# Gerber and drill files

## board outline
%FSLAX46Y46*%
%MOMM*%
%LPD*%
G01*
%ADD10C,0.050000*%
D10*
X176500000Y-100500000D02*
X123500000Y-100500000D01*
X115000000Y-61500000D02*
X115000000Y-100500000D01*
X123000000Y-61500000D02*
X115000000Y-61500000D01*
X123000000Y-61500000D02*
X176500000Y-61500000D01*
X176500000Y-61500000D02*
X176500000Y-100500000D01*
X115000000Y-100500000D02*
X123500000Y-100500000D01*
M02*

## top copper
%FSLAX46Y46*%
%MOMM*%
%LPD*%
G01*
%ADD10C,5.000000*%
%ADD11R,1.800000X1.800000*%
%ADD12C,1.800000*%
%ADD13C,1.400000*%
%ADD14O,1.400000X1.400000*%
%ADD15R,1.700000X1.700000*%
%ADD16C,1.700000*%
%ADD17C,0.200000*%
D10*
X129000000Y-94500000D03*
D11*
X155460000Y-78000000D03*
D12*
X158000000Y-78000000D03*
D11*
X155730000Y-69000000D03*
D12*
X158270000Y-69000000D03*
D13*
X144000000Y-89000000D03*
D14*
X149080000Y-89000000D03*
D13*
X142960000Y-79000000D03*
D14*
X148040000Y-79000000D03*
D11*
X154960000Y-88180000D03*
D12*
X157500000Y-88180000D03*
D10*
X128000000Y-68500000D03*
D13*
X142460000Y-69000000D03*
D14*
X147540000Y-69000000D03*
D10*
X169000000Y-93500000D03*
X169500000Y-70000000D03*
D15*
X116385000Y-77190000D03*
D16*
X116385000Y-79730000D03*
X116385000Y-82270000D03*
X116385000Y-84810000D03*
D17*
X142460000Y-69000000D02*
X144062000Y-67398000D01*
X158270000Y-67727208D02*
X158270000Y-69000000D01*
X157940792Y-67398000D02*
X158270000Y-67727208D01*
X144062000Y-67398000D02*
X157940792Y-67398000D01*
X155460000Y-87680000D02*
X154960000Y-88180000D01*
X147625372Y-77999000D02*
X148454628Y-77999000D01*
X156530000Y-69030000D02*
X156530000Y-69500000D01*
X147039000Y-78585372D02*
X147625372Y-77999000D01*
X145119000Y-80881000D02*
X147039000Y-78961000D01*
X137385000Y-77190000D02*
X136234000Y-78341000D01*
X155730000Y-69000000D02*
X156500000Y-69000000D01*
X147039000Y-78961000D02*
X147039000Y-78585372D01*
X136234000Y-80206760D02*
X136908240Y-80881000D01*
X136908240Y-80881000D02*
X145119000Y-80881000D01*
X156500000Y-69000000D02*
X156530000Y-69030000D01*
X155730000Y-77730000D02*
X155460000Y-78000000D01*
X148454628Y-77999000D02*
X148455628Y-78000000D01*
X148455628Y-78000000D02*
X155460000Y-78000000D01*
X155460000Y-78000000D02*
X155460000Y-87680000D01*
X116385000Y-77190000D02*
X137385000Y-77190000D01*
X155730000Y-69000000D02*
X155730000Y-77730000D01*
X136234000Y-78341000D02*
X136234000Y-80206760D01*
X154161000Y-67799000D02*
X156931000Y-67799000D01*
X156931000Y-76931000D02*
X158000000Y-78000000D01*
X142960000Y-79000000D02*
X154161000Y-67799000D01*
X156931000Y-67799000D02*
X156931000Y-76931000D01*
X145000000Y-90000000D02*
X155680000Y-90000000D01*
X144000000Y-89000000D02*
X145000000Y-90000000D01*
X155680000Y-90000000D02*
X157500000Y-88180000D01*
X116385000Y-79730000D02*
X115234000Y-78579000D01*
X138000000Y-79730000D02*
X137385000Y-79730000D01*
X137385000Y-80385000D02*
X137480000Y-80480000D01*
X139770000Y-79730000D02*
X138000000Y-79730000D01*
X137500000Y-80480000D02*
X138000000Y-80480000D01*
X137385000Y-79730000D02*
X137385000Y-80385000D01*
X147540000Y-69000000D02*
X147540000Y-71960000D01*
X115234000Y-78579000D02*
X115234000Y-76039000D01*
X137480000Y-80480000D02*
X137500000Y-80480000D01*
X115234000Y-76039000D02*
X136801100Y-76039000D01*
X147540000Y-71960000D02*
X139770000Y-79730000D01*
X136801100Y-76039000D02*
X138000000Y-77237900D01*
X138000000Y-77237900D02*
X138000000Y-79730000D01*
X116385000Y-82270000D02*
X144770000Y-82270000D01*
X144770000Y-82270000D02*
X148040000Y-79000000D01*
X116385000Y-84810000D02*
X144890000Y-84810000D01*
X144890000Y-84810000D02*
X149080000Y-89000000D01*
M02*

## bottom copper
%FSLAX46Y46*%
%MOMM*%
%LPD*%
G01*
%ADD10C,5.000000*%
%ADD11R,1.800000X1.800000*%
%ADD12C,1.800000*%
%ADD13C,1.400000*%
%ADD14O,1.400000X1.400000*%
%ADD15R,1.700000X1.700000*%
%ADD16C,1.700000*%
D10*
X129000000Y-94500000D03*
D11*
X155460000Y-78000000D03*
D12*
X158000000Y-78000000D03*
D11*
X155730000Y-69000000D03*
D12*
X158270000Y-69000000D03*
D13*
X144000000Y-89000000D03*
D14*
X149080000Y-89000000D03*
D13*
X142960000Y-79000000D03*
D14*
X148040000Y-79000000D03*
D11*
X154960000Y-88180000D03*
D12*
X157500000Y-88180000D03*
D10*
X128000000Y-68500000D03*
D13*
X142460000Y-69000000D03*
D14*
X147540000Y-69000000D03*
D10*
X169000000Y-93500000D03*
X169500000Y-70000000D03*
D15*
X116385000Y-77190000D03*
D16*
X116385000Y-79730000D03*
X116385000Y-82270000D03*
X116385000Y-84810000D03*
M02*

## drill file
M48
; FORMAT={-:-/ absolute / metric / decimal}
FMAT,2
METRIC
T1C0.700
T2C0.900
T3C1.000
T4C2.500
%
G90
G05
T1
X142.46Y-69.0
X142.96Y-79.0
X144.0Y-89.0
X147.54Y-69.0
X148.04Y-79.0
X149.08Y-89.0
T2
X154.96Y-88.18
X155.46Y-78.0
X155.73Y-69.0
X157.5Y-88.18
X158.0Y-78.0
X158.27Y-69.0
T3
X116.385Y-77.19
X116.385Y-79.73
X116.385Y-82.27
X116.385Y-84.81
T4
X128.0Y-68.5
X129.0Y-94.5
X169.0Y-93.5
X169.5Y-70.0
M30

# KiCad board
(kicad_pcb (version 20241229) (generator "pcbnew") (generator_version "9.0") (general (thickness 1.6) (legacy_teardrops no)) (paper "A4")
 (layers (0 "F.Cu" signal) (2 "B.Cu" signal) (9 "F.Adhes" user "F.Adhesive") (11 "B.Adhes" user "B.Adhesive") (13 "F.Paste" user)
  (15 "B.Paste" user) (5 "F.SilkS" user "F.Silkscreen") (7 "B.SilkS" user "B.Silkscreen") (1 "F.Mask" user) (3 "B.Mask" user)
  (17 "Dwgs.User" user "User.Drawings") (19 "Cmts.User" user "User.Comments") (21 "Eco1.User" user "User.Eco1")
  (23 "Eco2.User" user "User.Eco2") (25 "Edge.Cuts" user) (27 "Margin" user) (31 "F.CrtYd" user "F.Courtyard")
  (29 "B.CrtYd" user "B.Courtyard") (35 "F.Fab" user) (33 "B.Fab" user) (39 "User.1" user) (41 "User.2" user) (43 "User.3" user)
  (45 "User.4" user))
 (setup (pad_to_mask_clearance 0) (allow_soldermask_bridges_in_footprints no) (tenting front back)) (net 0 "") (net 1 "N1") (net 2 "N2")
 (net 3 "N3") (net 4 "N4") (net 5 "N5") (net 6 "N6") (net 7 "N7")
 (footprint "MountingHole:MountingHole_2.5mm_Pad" (layer "F.Cu") (at 129 94.5)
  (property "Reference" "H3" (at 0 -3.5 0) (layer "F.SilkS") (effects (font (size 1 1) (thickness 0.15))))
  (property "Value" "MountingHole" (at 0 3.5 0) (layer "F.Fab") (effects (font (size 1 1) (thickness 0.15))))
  (pad "1" thru_hole circle (at 0 0) (size 5 5) (drill 2.5) (layers "*.Cu" "*.Mask") (remove_unused_layers no)))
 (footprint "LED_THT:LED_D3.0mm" (layer "F.Cu") (at 155.46 78)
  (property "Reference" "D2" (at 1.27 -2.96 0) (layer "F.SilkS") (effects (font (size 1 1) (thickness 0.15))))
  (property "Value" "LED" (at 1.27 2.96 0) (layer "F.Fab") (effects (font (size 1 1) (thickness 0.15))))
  (pad "1" thru_hole rect (at 0 0) (size 1.8 1.8) (drill 0.9) (layers "*.Cu" "*.Mask") (remove_unused_layers no) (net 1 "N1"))
  (pad "2" thru_hole circle (at 2.54 0) (size 1.8 1.8) (drill 0.9) (layers "*.Cu" "*.Mask") (remove_unused_layers no) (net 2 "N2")))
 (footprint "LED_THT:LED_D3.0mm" (layer "F.Cu") (at 155.73 69)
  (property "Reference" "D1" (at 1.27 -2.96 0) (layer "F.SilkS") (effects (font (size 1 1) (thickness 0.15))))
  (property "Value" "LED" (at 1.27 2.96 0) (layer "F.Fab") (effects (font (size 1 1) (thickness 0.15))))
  (pad "1" thru_hole rect (at 0 0) (size 1.8 1.8) (drill 0.9) (layers "*.Cu" "*.Mask") (remove_unused_layers no) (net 1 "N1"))
  (pad "2" thru_hole circle (at 2.54 0) (size 1.8 1.8) (drill 0.9) (layers "*.Cu" "*.Mask") (remove_unused_layers no) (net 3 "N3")))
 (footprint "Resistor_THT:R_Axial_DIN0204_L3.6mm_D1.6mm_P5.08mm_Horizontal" (layer "F.Cu") (at 144 89)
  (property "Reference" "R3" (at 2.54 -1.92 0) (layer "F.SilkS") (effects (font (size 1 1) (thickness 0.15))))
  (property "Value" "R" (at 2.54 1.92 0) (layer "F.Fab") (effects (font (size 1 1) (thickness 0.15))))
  (pad "1" thru_hole circle (at 0 0) (size 1.4 1.4) (drill 0.7) (layers "*.Cu" "*.Mask") (remove_unused_layers no) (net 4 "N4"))
  (pad "2" thru_hole oval (at 5.08 0) (size 1.4 1.4) (drill 0.7) (layers "*.Cu" "*.Mask") (remove_unused_layers no) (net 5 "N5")))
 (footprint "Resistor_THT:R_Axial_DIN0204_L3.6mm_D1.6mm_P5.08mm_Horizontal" (layer "F.Cu") (at 142.96 79)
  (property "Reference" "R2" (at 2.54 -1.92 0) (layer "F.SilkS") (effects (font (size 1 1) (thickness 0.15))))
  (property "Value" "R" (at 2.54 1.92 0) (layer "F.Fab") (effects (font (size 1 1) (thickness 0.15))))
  (pad "1" thru_hole circle (at 0 0) (size 1.4 1.4) (drill 0.7) (layers "*.Cu" "*.Mask") (remove_unused_layers no) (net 2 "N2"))
  (pad "2" thru_hole oval (at 5.08 0) (size 1.4 1.4) (drill 0.7) (layers "*.Cu" "*.Mask") (remove_unused_layers no) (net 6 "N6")))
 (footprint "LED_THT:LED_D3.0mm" (layer "F.Cu") (at 154.96 88.18)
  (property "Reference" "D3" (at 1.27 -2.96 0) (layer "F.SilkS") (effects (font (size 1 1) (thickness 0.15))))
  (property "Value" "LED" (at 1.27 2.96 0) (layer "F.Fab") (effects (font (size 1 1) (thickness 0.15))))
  (pad "1" thru_hole rect (at 0 0) (size 1.8 1.8) (drill 0.9) (layers "*.Cu" "*.Mask") (remove_unused_layers no) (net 1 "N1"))
  (pad "2" thru_hole circle (at 2.54 0) (size 1.8 1.8) (drill 0.9) (layers "*.Cu" "*.Mask") (remove_unused_layers no) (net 4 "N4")))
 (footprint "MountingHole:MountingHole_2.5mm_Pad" (layer "F.Cu") (at 128 68.5)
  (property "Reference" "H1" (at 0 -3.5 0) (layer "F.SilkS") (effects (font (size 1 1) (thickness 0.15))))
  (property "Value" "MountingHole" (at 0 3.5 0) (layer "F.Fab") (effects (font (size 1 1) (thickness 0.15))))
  (pad "1" thru_hole circle (at 0 0) (size 5 5) (drill 2.5) (layers "*.Cu" "*.Mask") (remove_unused_layers no)))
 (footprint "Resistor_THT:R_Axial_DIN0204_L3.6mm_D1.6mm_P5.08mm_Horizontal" (layer "F.Cu") (at 142.46 69)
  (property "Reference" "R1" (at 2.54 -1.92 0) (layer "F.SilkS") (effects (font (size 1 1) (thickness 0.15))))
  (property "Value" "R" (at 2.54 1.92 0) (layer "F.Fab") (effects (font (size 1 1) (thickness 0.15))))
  (pad "1" thru_hole circle (at 0 0) (size 1.4 1.4) (drill 0.7) (layers "*.Cu" "*.Mask") (remove_unused_layers no) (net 3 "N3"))
  (pad "2" thru_hole oval (at 5.08 0) (size 1.4 1.4) (drill 0.7) (layers "*.Cu" "*.Mask") (remove_unused_layers no) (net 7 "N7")))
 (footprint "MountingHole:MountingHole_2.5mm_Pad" (layer "F.Cu") (at 169 93.5)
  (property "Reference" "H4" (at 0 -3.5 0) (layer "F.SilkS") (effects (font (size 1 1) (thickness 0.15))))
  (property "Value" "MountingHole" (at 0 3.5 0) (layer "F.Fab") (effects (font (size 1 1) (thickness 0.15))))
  (pad "1" thru_hole circle (at 0 0) (size 5 5) (drill 2.5) (layers "*.Cu" "*.Mask") (remove_unused_layers no)))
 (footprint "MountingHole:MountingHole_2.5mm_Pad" (layer "F.Cu") (at 169.5 70)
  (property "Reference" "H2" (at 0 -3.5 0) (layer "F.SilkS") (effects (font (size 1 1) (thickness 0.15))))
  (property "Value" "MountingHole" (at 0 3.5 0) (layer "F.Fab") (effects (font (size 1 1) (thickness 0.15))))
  (pad "1" thru_hole circle (at 0 0) (size 5 5) (drill 2.5) (layers "*.Cu" "*.Mask") (remove_unused_layers no)))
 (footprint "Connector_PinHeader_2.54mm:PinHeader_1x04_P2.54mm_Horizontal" (layer "B.Cu") (at 116.385 77.19 180)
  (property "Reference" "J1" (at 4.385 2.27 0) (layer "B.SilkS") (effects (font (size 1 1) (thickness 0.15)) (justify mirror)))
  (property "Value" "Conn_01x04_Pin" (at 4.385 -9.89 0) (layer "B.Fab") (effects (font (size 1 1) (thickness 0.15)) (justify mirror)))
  (pad "1" thru_hole rect (at 0 0 180) (size 1.7 1.7) (drill 1) (layers "*.Cu" "*.Mask") (remove_unused_layers no) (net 1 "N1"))
  (pad "2" thru_hole circle (at 0 -2.54 180) (size 1.7 1.7) (drill 1) (layers "*.Cu" "*.Mask") (remove_unused_layers no) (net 7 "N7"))
  (pad "3" thru_hole circle (at 0 -5.08 180) (size 1.7 1.7) (drill 1) (layers "*.Cu" "*.Mask") (remove_unused_layers no) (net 6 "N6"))
  (pad "4" thru_hole circle (at 0 -7.62 180) (size 1.7 1.7) (drill 1) (layers "*.Cu" "*.Mask") (remove_unused_layers no) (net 5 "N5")))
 (gr_line (start 176.5 100.5) (end 123.5 100.5) (stroke (width 0.05) (type default)) (layer "Edge.Cuts"))
 (gr_line (start 115 61.5) (end 115 100.5) (stroke (width 0.05) (type default)) (layer "Edge.Cuts"))
 (gr_line (start 123 61.5) (end 115 61.5) (stroke (width 0.05) (type default)) (layer "Edge.Cuts"))
 (gr_line (start 123 61.5) (end 176.5 61.5) (stroke (width 0.05) (type default)) (layer "Edge.Cuts"))
 (gr_line (start 176.5 61.5) (end 176.5 100.5) (stroke (width 0.05) (type default)) (layer "Edge.Cuts"))
 (gr_line (start 115 100.5) (end 123.5 100.5) (stroke (width 0.05) (type default)) (layer "Edge.Cuts"))
 (segment (start 142.46 69) (end 144.062 67.398) (width 0.2) (layer "F.Cu") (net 3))
 (segment (start 158.27 67.727208) (end 158.27 69) (width 0.2) (layer "F.Cu") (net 3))
 (segment (start 157.940792 67.398) (end 158.27 67.727208) (width 0.2) (layer "F.Cu") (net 3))
 (segment (start 144.062 67.398) (end 157.940792 67.398) (width 0.2) (layer "F.Cu") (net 3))
 (segment (start 155.46 87.68) (end 154.96 88.18) (width 0.2) (layer "F.Cu") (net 1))
 (segment (start 147.625372 77.999) (end 148.454628 77.999) (width 0.2) (layer "F.Cu") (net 1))
 (segment (start 156.53 69.03) (end 156.53 69.5) (width 0.2) (layer "F.Cu") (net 1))
 (segment (start 147.039 78.585372) (end 147.625372 77.999) (width 0.2) (layer "F.Cu") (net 1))
 (segment (start 145.119 80.881) (end 147.039 78.961) (width 0.2) (layer "F.Cu") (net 1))
 (segment (start 137.385 77.19) (end 136.234 78.341) (width 0.2) (layer "F.Cu") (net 1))
 (segment (start 155.73 69) (end 156.5 69) (width 0.2) (layer "F.Cu") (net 1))
 (segment (start 147.039 78.961) (end 147.039 78.585372) (width 0.2) (layer "F.Cu") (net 1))
 (segment (start 136.234 80.20676) (end 136.90824 80.881) (width 0.2) (layer "F.Cu") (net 1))
 (segment (start 136.90824 80.881) (end 145.119 80.881) (width 0.2) (layer "F.Cu") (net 1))
 (segment (start 156.5 69) (end 156.53 69.03) (width 0.2) (layer "F.Cu") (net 1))
 (segment (start 155.73 77.73) (end 155.46 78) (width 0.2) (layer "F.Cu") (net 1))
 (segment (start 148.454628 77.999) (end 148.455628 78) (width 0.2) (layer "F.Cu") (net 1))
 (segment (start 148.455628 78) (end 155.46 78) (width 0.2) (layer "F.Cu") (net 1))
 (segment (start 155.46 78) (end 155.46 87.68) (width 0.2) (layer "F.Cu") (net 1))
 (segment (start 116.385 77.19) (end 137.385 77.19) (width 0.2) (layer "F.Cu") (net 1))
 (segment (start 155.73 69) (end 155.73 77.73) (width 0.2) (layer "F.Cu") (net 1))
 (segment (start 136.234 78.341) (end 136.234 80.20676) (width 0.2) (layer "F.Cu") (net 1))
 (segment (start 154.161 67.799) (end 156.931 67.799) (width 0.2) (layer "F.Cu") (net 2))
 (segment (start 156.931 76.931) (end 158 78) (width 0.2) (layer "F.Cu") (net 2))
 (segment (start 142.96 79) (end 154.161 67.799) (width 0.2) (layer "F.Cu") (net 2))
 (segment (start 156.931 67.799) (end 156.931 76.931) (width 0.2) (layer "F.Cu") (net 2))
 (segment (start 145 90) (end 155.68 90) (width 0.2) (layer "F.Cu") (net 4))
 (segment (start 144 89) (end 145 90) (width 0.2) (layer "F.Cu") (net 4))
 (segment (start 155.68 90) (end 157.5 88.18) (width 0.2) (layer "F.Cu") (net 4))
 (segment (start 116.385 79.73) (end 115.234 78.579) (width 0.2) (layer "F.Cu") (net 7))
 (segment (start 138 79.73) (end 137.385 79.73) (width 0.2) (layer "F.Cu") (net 7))
 (segment (start 137.385 80.385) (end 137.48 80.48) (width 0.2) (layer "F.Cu") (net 7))
 (segment (start 139.77 79.73) (end 138 79.73) (width 0.2) (layer "F.Cu") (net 7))
 (segment (start 137.5 80.48) (end 138 80.48) (width 0.2) (layer "F.Cu") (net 7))
 (segment (start 137.385 79.73) (end 137.385 80.385) (width 0.2) (layer "F.Cu") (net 7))
 (segment (start 147.54 69) (end 147.54 71.96) (width 0.2) (layer "F.Cu") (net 7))
 (segment (start 115.234 78.579) (end 115.234 76.039) (width 0.2) (layer "F.Cu") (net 7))
 (segment (start 137.48 80.48) (end 137.5 80.48) (width 0.2) (layer "F.Cu") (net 7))
 (segment (start 115.234 76.039) (end 136.8011 76.039) (width 0.2) (layer "F.Cu") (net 7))
 (segment (start 147.54 71.96) (end 139.77 79.73) (width 0.2) (layer "F.Cu") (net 7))
 (segment (start 136.8011 76.039) (end 138 77.2379) (width 0.2) (layer "F.Cu") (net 7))
 (segment (start 138 77.2379) (end 138 79.73) (width 0.2) (layer "F.Cu") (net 7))
 (segment (start 116.385 82.27) (end 144.77 82.27) (width 0.2) (layer "F.Cu") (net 6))
 (segment (start 144.77 82.27) (end 148.04 79) (width 0.2) (layer "F.Cu") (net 6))
 (segment (start 116.385 84.81) (end 144.89 84.81) (width 0.2) (layer "F.Cu") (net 5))
 (segment (start 144.89 84.81) (end 149.08 89) (width 0.2) (layer "F.Cu") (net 5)))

